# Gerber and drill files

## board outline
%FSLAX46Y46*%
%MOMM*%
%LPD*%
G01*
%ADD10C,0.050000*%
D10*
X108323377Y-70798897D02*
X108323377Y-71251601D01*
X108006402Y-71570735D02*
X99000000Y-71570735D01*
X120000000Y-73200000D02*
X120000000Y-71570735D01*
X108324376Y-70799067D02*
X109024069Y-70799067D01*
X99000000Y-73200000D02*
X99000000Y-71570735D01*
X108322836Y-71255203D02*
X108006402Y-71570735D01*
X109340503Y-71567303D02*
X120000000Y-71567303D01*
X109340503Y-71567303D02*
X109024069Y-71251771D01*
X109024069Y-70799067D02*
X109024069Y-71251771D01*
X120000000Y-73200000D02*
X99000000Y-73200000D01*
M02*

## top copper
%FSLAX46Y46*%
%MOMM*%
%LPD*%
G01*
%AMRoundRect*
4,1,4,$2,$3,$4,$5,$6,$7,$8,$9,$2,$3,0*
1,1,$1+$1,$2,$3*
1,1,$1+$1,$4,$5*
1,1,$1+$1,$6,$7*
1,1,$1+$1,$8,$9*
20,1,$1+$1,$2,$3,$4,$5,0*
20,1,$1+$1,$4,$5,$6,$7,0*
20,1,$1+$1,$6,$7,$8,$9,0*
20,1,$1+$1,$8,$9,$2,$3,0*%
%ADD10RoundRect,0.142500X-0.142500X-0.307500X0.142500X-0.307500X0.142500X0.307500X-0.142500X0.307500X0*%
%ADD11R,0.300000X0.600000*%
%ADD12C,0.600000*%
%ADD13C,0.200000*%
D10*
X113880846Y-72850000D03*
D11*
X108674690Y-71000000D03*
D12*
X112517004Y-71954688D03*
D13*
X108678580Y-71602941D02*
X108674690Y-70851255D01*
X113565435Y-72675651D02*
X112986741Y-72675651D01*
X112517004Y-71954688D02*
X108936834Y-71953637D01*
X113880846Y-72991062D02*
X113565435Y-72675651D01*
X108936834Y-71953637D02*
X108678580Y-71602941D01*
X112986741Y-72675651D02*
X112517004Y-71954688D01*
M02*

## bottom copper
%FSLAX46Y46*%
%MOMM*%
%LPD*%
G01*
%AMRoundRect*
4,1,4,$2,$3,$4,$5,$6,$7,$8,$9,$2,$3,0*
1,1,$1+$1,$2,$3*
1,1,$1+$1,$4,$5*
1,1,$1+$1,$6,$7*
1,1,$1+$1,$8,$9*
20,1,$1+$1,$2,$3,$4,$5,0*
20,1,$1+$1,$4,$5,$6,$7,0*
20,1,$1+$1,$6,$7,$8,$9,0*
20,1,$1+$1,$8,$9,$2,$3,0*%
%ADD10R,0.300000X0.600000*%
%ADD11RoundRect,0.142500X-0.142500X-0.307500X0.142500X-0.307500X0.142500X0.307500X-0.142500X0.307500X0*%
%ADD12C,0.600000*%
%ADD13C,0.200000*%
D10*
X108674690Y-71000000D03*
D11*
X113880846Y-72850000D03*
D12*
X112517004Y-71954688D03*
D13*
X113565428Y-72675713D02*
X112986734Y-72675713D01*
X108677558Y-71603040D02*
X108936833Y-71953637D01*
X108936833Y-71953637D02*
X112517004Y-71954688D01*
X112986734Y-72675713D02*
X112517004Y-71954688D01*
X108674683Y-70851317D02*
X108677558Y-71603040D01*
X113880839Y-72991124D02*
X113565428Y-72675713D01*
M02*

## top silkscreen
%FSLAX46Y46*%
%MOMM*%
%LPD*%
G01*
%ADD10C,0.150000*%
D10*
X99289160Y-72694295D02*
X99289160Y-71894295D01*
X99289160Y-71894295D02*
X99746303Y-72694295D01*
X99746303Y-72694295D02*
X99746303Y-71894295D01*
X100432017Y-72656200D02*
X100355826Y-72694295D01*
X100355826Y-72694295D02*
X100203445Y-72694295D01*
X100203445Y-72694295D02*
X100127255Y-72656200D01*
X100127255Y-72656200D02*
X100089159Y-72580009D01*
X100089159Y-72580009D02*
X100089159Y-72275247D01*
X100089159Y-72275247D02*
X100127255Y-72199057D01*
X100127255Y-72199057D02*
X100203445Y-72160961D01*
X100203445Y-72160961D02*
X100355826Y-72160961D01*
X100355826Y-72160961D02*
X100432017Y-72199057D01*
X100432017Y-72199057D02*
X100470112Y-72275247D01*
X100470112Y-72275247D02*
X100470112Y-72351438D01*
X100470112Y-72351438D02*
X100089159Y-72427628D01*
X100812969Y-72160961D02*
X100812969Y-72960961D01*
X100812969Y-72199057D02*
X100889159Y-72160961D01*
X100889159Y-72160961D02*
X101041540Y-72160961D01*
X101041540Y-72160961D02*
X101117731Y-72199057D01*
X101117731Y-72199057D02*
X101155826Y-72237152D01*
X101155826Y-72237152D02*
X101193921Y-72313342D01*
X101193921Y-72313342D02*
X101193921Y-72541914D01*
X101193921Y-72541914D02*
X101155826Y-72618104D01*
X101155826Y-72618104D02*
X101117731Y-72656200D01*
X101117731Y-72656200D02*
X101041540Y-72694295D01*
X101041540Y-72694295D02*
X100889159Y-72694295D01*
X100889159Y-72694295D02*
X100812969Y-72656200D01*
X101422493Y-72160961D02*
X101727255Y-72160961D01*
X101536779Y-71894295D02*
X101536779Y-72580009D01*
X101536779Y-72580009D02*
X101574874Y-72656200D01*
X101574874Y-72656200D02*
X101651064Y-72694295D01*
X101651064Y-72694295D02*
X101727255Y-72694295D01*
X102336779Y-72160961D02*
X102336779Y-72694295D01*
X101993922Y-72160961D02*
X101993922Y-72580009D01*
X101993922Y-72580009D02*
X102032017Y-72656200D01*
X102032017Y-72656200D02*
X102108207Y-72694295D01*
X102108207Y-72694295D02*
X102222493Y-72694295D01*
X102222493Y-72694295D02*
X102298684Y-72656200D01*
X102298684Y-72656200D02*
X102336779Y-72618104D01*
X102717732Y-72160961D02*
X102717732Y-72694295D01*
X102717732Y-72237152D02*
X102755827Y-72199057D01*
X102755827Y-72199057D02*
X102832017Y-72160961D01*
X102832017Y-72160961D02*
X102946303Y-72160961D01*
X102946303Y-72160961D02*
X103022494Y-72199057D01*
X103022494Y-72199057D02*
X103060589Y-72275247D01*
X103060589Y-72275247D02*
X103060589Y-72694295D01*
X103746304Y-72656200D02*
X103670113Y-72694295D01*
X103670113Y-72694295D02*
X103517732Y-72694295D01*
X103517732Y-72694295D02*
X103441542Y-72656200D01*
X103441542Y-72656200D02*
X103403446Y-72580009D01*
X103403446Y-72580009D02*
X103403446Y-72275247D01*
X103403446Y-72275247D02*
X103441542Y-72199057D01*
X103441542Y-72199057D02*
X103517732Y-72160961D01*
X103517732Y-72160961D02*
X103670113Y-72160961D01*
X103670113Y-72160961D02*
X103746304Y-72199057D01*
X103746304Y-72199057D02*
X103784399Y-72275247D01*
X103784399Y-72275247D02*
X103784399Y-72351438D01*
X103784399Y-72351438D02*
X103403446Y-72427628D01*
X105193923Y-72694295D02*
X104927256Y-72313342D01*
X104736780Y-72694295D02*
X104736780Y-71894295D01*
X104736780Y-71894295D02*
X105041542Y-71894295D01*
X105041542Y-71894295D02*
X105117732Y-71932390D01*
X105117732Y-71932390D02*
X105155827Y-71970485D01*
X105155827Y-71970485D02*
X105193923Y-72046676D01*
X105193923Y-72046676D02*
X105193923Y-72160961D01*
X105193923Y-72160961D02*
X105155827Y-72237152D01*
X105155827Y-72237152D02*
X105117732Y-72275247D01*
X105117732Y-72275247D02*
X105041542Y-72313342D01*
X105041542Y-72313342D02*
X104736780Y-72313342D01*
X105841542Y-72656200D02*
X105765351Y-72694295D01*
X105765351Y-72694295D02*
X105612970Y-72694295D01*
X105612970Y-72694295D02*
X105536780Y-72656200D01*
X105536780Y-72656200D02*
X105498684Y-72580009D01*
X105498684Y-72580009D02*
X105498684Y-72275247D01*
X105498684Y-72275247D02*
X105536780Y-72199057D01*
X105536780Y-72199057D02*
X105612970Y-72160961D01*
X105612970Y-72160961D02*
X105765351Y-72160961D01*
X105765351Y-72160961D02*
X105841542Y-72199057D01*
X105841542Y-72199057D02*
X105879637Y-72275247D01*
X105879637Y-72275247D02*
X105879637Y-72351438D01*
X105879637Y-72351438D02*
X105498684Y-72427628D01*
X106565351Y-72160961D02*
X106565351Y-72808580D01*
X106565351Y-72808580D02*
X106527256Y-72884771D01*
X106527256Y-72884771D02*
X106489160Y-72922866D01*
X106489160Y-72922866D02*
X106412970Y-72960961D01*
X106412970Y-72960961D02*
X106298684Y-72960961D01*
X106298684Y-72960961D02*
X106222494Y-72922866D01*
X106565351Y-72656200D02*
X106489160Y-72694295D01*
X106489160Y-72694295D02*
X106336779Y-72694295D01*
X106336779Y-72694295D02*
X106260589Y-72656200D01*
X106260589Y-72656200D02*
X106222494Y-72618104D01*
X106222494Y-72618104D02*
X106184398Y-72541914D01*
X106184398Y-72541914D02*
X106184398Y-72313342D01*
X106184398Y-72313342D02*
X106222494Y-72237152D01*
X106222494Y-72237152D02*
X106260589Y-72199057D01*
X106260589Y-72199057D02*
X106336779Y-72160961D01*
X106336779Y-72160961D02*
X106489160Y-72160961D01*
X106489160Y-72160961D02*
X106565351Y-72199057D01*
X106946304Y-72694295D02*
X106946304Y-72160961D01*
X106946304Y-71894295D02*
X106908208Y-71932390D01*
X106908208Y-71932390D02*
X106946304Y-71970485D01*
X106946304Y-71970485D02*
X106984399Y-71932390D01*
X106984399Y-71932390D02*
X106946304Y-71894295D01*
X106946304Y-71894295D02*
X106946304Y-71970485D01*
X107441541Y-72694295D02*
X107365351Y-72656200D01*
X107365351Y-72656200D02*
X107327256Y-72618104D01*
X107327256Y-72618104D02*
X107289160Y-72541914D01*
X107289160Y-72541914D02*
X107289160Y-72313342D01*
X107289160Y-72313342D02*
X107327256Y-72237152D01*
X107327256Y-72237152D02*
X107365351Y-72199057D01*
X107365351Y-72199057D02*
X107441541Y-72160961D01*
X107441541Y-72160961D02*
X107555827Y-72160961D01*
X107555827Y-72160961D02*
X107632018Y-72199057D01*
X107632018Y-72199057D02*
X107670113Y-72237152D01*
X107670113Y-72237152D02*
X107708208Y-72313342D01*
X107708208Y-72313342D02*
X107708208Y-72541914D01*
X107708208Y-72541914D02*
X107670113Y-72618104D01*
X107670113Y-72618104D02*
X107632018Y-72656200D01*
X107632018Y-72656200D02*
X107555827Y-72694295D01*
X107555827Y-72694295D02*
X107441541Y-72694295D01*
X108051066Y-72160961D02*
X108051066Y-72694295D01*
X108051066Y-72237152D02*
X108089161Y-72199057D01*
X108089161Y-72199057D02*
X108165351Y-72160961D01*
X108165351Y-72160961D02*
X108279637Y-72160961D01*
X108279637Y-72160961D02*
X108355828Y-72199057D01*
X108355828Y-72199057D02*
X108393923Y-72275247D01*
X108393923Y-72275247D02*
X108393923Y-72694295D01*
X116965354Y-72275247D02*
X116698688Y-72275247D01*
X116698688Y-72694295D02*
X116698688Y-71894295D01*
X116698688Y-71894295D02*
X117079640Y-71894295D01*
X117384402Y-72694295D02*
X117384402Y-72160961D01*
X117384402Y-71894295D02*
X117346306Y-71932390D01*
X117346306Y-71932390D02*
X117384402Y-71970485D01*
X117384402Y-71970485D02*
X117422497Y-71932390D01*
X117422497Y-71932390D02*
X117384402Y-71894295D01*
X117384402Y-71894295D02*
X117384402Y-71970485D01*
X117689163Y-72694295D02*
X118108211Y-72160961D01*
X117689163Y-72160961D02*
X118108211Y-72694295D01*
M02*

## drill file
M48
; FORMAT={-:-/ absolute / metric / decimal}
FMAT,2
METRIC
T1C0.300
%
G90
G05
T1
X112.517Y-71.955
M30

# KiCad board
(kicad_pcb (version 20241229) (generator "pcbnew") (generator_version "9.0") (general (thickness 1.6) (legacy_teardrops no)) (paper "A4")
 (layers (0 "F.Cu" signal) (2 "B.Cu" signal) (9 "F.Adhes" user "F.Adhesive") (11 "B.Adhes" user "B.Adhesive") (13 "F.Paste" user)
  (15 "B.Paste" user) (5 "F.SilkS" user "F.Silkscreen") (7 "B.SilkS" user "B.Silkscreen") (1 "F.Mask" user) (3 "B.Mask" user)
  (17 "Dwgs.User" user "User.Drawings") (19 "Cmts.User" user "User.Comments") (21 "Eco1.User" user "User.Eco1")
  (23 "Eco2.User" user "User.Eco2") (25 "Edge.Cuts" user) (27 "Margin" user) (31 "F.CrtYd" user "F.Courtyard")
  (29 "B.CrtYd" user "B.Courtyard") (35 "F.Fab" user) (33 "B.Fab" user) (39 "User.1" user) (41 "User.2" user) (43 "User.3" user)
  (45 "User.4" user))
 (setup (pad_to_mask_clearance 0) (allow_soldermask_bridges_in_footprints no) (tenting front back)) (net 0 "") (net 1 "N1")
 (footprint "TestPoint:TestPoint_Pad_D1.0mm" (layer "F.Cu") (at 113.880846 72.991062)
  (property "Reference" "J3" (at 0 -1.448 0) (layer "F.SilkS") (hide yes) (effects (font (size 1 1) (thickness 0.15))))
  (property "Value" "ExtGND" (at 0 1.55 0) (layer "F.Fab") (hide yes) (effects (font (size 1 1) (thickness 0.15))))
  (pad "1" smd roundrect (at 0 -0.141062) (size 0.57 0.9) (layers "F.Cu" "F.Mask" "F.Paste") (roundrect_rratio 0.25) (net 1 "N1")
   (thermal_bridge_angle 45)))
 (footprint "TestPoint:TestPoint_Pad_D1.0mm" (layer "F.Cu") (at 108.67469 70.851255)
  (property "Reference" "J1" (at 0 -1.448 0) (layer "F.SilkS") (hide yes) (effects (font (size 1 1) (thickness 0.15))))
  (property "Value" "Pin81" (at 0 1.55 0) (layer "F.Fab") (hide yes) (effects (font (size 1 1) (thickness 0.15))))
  (pad "1" smd rect (at 0 0.148745) (size 0.3 0.6) (layers "F.Cu" "F.Mask" "F.Paste") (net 1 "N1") (thermal_bridge_angle 45)))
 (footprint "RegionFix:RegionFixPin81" (layer "B.Cu") (at 108.701945 70.852727)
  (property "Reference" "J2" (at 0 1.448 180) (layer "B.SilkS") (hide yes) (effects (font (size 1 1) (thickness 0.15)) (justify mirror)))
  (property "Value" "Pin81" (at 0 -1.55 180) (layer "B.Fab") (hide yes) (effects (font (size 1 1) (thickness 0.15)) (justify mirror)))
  (pad "1" smd rect (at -0.027255 0.147273) (size 0.3 0.6) (layers "B.Cu" "B.Mask" "B.Paste") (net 1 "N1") (thermal_bridge_angle 45)))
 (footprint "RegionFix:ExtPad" (layer "B.Cu") (at 113.908775 72.993199)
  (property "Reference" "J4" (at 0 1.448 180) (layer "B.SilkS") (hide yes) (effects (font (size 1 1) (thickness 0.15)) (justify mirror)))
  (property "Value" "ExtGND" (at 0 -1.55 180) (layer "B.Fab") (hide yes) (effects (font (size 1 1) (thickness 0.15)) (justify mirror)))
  (pad "1" smd roundrect (at -0.027929 -0.143199) (size 0.57 0.9) (layers "B.Cu" "B.Mask" "B.Paste") (roundrect_rratio 0.25) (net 1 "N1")
   (thermal_bridge_angle 45)))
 (gr_line (start 108.323377 70.798897) (end 108.323377 71.251601) (stroke (width 0.05) (type default)) (layer "Edge.Cuts"))
 (gr_line (start 108.006402 71.570735) (end 99 71.570735) (stroke (width 0.05) (type default)) (layer "Edge.Cuts"))
 (gr_line (start 120 73.2) (end 120 71.570735) (stroke (width 0.05) (type default)) (layer "Edge.Cuts"))
 (gr_line (start 108.324376 70.799067) (end 109.024069 70.799067) (stroke (width 0.05) (type default)) (layer "Edge.Cuts"))
 (gr_line (start 99 73.2) (end 99 71.570735) (stroke (width 0.05) (type default)) (layer "Edge.Cuts"))
 (gr_line (start 108.322836 71.255203) (end 108.006402 71.570735) (stroke (width 0.05) (type default)) (layer "Edge.Cuts"))
 (gr_line (start 109.340503 71.567303) (end 120 71.567303) (stroke (width 0.05) (type default)) (layer "Edge.Cuts"))
 (gr_line (start 109.340503 71.567303) (end 109.024069 71.251771) (stroke (width 0.05) (type default)) (layer "Edge.Cuts"))
 (gr_line (start 109.024069 70.799067) (end 109.024069 71.251771) (stroke (width 0.05) (type default)) (layer "Edge.Cuts"))
 (gr_line (start 120 73.2) (end 99 73.2) (stroke (width 0.05) (type default)) (layer "Edge.Cuts"))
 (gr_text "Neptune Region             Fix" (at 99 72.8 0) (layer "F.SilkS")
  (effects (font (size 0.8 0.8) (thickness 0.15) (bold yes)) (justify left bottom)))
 (segment (start 108.67858 71.602941) (end 108.67469 70.851255) (width 0.2) (layer "F.Cu") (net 1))
 (segment (start 113.565435 72.675651) (end 112.986741 72.675651) (width 0.2) (layer "F.Cu") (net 1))
 (segment (start 112.517004 71.954688) (end 108.936834 71.953637) (width 0.2) (layer "F.Cu") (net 1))
 (segment (start 113.880846 72.991062) (end 113.565435 72.675651) (width 0.2) (layer "F.Cu") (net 1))
 (segment (start 108.936834 71.953637) (end 108.67858 71.602941) (width 0.2) (layer "F.Cu") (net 1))
 (segment (start 112.986741 72.675651) (end 112.517004 71.954688) (width 0.2) (layer "F.Cu") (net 1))
 (via (at 112.517004 71.954688) (size 0.6) (drill 0.3) (layers "F.Cu" "B.Cu") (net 1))
 (segment (start 113.565428 72.675713) (end 112.986734 72.675713) (width 0.2) (layer "B.Cu") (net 1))
 (segment (start 108.677558 71.60304) (end 108.936833 71.953637) (width 0.2) (layer "B.Cu") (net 1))
 (segment (start 108.936833 71.953637) (end 112.517004 71.954688) (width 0.2) (layer "B.Cu") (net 1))
 (segment (start 112.986734 72.675713) (end 112.517004 71.954688) (width 0.2) (layer "B.Cu") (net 1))
 (segment (start 108.674683 70.851317) (end 108.677558 71.60304) (width 0.2) (layer "B.Cu") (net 1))
 (segment (start 113.880839 72.991124) (end 113.565428 72.675713) (width 0.2) (layer "B.Cu") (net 1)))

